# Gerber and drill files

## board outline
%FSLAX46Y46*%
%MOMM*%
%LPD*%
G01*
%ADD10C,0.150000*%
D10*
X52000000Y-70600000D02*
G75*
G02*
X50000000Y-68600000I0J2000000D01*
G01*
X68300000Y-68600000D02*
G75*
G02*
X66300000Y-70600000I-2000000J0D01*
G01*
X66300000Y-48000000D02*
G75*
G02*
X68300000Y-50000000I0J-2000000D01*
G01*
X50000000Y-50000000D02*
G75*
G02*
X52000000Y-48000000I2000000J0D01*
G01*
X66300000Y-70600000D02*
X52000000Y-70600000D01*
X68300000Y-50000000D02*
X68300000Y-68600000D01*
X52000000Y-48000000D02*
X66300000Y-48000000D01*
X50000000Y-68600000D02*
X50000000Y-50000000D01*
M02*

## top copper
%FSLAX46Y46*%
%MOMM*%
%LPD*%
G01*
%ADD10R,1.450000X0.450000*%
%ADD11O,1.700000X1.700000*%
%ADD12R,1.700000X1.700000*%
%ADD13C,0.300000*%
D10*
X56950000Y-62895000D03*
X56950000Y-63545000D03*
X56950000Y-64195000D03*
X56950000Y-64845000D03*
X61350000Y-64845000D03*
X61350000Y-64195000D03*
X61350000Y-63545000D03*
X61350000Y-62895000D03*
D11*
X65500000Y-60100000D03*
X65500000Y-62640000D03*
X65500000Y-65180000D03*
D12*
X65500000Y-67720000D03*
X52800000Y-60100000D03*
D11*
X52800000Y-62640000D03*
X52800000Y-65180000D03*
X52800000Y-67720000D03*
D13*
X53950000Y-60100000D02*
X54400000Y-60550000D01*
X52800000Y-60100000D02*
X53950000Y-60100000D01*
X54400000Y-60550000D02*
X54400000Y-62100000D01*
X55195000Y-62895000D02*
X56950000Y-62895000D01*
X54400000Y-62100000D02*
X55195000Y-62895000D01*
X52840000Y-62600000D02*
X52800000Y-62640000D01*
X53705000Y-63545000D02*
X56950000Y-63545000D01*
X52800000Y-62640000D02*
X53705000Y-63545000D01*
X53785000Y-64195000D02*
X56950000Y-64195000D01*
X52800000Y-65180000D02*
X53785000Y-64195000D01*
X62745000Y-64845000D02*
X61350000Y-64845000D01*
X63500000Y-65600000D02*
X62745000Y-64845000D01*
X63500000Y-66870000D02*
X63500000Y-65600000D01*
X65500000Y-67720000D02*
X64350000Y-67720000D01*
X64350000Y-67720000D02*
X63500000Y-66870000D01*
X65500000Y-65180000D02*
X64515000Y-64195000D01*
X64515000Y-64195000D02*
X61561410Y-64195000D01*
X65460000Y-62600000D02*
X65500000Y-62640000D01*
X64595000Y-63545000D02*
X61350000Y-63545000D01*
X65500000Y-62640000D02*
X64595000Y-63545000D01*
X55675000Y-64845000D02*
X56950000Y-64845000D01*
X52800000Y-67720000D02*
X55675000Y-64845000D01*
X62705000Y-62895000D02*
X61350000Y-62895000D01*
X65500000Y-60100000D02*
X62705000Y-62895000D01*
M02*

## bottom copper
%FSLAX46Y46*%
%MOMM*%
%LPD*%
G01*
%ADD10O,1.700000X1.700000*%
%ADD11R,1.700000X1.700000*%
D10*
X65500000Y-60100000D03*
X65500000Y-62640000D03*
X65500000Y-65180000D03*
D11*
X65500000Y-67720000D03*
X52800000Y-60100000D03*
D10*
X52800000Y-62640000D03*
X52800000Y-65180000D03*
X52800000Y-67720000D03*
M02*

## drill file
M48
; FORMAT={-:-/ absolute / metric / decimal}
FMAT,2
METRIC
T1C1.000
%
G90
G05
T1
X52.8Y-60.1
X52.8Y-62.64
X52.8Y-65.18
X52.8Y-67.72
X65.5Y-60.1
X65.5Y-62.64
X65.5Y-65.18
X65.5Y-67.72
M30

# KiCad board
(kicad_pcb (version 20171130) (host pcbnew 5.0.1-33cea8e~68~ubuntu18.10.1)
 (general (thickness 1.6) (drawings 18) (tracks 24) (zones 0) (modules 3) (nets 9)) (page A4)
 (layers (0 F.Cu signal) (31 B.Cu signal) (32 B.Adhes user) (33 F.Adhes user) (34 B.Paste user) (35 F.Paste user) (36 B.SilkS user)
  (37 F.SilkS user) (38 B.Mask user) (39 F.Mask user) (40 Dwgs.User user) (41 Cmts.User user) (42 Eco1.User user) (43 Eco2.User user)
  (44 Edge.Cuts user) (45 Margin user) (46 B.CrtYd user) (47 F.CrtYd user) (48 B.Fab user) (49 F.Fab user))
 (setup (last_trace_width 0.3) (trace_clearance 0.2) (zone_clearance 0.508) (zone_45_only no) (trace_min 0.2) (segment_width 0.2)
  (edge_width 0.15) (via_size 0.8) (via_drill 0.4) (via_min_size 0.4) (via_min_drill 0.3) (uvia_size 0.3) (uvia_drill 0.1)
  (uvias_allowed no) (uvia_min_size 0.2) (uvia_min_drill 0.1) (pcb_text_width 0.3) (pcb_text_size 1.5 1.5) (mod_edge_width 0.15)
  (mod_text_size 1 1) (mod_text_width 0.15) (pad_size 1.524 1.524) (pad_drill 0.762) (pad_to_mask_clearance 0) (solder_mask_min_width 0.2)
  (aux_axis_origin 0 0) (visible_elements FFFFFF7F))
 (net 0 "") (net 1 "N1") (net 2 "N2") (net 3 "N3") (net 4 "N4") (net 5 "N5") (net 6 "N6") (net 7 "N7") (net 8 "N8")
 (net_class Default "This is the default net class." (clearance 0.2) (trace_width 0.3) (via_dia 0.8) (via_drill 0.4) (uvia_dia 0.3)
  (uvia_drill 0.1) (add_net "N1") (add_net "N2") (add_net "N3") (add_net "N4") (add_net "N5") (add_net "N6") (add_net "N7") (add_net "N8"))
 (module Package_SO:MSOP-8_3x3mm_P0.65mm (layer F.Cu) (at 59.15 63.87)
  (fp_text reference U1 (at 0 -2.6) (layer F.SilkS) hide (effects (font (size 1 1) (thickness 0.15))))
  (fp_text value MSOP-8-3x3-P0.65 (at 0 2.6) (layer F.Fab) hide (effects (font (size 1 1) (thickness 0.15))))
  (pad 1 smd rect (at -2.2 -0.975) (size 1.45 0.45) (layers F.Cu F.Paste F.Mask) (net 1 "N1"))
  (pad 2 smd rect (at -2.2 -0.325) (size 1.45 0.45) (layers F.Cu F.Paste F.Mask) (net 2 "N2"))
  (pad 3 smd rect (at -2.2 0.325) (size 1.45 0.45) (layers F.Cu F.Paste F.Mask) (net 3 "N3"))
  (pad 4 smd rect (at -2.2 0.975) (size 1.45 0.45) (layers F.Cu F.Paste F.Mask) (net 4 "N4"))
  (pad 5 smd rect (at 2.2 0.975) (size 1.45 0.45) (layers F.Cu F.Paste F.Mask) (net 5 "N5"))
  (pad 6 smd rect (at 2.2 0.325) (size 1.45 0.45) (layers F.Cu F.Paste F.Mask) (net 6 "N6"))
  (pad 7 smd rect (at 2.2 -0.325) (size 1.45 0.45) (layers F.Cu F.Paste F.Mask) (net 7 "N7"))
  (pad 8 smd rect (at 2.2 -0.975) (size 1.45 0.45) (layers F.Cu F.Paste F.Mask) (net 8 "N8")))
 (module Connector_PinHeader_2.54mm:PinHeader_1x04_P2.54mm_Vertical (layer F.Cu) (at 65.5 67.72 180)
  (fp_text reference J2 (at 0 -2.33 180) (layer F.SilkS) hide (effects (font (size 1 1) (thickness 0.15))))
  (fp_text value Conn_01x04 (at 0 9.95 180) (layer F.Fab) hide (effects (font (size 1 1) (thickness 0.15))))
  (pad 4 thru_hole oval (at 0 7.62 180) (size 1.7 1.7) (drill 1) (layers *.Cu *.Mask) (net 8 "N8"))
  (pad 3 thru_hole oval (at 0 5.08 180) (size 1.7 1.7) (drill 1) (layers *.Cu *.Mask) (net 7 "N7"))
  (pad 2 thru_hole oval (at 0 2.54 180) (size 1.7 1.7) (drill 1) (layers *.Cu *.Mask) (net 6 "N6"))
  (pad 1 thru_hole rect (at 0 0 180) (size 1.7 1.7) (drill 1) (layers *.Cu *.Mask) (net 5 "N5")))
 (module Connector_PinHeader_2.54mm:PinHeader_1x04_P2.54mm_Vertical (layer F.Cu) (at 52.8 60.1)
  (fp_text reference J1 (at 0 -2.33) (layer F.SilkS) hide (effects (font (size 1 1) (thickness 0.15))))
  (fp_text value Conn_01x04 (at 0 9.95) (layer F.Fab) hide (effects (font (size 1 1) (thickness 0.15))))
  (pad 1 thru_hole rect (at 0 0) (size 1.7 1.7) (drill 1) (layers *.Cu *.Mask) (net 1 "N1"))
  (pad 2 thru_hole oval (at 0 2.54) (size 1.7 1.7) (drill 1) (layers *.Cu *.Mask) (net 2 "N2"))
  (pad 3 thru_hole oval (at 0 5.08) (size 1.7 1.7) (drill 1) (layers *.Cu *.Mask) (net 3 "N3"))
  (pad 4 thru_hole oval (at 0 7.62) (size 1.7 1.7) (drill 1) (layers *.Cu *.Mask) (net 4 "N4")))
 (gr_arc (start 52 68.6) (end 50 68.6) (angle -90) (layer Edge.Cuts) (width 0.15))
 (gr_arc (start 66.3 68.6) (end 66.3 70.6) (angle -90) (layer Edge.Cuts) (width 0.15))
 (gr_arc (start 66.3 50) (end 68.3 50) (angle -90) (layer Edge.Cuts) (width 0.15))
 (gr_arc (start 52 50) (end 52 48) (angle -90) (layer Edge.Cuts) (width 0.15))
 (gr_line (start 66.3 70.6) (end 52 70.6) (layer Edge.Cuts) (width 0.15))
 (gr_line (start 68.3 50) (end 68.3 68.6) (layer Edge.Cuts) (width 0.15))
 (gr_line (start 52 48) (end 66.3 48) (layer Edge.Cuts) (width 0.15))
 (gr_line (start 50 68.6) (end 50 50) (layer Edge.Cuts) (width 0.15))
 (segment (start 53.95 60.1) (end 54.4 60.55) (width 0.3) (layer F.Cu) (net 1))
 (segment (start 52.8 60.1) (end 53.95 60.1) (width 0.3) (layer F.Cu) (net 1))
 (segment (start 54.4 60.55) (end 54.4 62.1) (width 0.3) (layer F.Cu) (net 1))
 (segment (start 55.195 62.895) (end 56.95 62.895) (width 0.3) (layer F.Cu) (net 1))
 (segment (start 54.4 62.1) (end 55.195 62.895) (width 0.3) (layer F.Cu) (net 1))
 (segment (start 52.84 62.6) (end 52.8 62.64) (width 0.3) (layer F.Cu) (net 2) (status 30))
 (segment (start 53.705 63.545) (end 56.95 63.545) (width 0.3) (layer F.Cu) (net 2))
 (segment (start 52.8 62.64) (end 53.705 63.545) (width 0.3) (layer F.Cu) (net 2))
 (segment (start 53.785 64.195) (end 56.95 64.195) (width 0.3) (layer F.Cu) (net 3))
 (segment (start 52.8 65.18) (end 53.785 64.195) (width 0.3) (layer F.Cu) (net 3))
 (segment (start 62.745 64.845) (end 61.35 64.845) (width 0.3) (layer F.Cu) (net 5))
 (segment (start 63.5 65.6) (end 62.745 64.845) (width 0.3) (layer F.Cu) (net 5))
 (segment (start 63.5 66.87) (end 63.5 65.6) (width 0.3) (layer F.Cu) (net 5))
 (segment (start 65.5 67.72) (end 64.35 67.72) (width 0.3) (layer F.Cu) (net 5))
 (segment (start 64.35 67.72) (end 63.5 66.87) (width 0.3) (layer F.Cu) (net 5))
 (segment (start 65.5 65.18) (end 64.515 64.195) (width 0.3) (layer F.Cu) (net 6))
 (segment (start 64.515 64.195) (end 61.56141 64.195) (width 0.3) (layer F.Cu) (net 6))
 (segment (start 65.46 62.6) (end 65.5 62.64) (width 0.3) (layer F.Cu) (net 7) (status 30))
 (segment (start 64.595 63.545) (end 61.35 63.545) (width 0.3) (layer F.Cu) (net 7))
 (segment (start 65.5 62.64) (end 64.595 63.545) (width 0.3) (layer F.Cu) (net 7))
 (segment (start 55.675 64.845) (end 56.95 64.845) (width 0.3) (layer F.Cu) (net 4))
 (segment (start 52.8 67.72) (end 55.675 64.845) (width 0.3) (layer F.Cu) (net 4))
 (segment (start 62.705 62.895) (end 61.35 62.895) (width 0.3) (layer F.Cu) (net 8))
 (segment (start 65.5 60.1) (end 62.705 62.895) (width 0.3) (layer F.Cu) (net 8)))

